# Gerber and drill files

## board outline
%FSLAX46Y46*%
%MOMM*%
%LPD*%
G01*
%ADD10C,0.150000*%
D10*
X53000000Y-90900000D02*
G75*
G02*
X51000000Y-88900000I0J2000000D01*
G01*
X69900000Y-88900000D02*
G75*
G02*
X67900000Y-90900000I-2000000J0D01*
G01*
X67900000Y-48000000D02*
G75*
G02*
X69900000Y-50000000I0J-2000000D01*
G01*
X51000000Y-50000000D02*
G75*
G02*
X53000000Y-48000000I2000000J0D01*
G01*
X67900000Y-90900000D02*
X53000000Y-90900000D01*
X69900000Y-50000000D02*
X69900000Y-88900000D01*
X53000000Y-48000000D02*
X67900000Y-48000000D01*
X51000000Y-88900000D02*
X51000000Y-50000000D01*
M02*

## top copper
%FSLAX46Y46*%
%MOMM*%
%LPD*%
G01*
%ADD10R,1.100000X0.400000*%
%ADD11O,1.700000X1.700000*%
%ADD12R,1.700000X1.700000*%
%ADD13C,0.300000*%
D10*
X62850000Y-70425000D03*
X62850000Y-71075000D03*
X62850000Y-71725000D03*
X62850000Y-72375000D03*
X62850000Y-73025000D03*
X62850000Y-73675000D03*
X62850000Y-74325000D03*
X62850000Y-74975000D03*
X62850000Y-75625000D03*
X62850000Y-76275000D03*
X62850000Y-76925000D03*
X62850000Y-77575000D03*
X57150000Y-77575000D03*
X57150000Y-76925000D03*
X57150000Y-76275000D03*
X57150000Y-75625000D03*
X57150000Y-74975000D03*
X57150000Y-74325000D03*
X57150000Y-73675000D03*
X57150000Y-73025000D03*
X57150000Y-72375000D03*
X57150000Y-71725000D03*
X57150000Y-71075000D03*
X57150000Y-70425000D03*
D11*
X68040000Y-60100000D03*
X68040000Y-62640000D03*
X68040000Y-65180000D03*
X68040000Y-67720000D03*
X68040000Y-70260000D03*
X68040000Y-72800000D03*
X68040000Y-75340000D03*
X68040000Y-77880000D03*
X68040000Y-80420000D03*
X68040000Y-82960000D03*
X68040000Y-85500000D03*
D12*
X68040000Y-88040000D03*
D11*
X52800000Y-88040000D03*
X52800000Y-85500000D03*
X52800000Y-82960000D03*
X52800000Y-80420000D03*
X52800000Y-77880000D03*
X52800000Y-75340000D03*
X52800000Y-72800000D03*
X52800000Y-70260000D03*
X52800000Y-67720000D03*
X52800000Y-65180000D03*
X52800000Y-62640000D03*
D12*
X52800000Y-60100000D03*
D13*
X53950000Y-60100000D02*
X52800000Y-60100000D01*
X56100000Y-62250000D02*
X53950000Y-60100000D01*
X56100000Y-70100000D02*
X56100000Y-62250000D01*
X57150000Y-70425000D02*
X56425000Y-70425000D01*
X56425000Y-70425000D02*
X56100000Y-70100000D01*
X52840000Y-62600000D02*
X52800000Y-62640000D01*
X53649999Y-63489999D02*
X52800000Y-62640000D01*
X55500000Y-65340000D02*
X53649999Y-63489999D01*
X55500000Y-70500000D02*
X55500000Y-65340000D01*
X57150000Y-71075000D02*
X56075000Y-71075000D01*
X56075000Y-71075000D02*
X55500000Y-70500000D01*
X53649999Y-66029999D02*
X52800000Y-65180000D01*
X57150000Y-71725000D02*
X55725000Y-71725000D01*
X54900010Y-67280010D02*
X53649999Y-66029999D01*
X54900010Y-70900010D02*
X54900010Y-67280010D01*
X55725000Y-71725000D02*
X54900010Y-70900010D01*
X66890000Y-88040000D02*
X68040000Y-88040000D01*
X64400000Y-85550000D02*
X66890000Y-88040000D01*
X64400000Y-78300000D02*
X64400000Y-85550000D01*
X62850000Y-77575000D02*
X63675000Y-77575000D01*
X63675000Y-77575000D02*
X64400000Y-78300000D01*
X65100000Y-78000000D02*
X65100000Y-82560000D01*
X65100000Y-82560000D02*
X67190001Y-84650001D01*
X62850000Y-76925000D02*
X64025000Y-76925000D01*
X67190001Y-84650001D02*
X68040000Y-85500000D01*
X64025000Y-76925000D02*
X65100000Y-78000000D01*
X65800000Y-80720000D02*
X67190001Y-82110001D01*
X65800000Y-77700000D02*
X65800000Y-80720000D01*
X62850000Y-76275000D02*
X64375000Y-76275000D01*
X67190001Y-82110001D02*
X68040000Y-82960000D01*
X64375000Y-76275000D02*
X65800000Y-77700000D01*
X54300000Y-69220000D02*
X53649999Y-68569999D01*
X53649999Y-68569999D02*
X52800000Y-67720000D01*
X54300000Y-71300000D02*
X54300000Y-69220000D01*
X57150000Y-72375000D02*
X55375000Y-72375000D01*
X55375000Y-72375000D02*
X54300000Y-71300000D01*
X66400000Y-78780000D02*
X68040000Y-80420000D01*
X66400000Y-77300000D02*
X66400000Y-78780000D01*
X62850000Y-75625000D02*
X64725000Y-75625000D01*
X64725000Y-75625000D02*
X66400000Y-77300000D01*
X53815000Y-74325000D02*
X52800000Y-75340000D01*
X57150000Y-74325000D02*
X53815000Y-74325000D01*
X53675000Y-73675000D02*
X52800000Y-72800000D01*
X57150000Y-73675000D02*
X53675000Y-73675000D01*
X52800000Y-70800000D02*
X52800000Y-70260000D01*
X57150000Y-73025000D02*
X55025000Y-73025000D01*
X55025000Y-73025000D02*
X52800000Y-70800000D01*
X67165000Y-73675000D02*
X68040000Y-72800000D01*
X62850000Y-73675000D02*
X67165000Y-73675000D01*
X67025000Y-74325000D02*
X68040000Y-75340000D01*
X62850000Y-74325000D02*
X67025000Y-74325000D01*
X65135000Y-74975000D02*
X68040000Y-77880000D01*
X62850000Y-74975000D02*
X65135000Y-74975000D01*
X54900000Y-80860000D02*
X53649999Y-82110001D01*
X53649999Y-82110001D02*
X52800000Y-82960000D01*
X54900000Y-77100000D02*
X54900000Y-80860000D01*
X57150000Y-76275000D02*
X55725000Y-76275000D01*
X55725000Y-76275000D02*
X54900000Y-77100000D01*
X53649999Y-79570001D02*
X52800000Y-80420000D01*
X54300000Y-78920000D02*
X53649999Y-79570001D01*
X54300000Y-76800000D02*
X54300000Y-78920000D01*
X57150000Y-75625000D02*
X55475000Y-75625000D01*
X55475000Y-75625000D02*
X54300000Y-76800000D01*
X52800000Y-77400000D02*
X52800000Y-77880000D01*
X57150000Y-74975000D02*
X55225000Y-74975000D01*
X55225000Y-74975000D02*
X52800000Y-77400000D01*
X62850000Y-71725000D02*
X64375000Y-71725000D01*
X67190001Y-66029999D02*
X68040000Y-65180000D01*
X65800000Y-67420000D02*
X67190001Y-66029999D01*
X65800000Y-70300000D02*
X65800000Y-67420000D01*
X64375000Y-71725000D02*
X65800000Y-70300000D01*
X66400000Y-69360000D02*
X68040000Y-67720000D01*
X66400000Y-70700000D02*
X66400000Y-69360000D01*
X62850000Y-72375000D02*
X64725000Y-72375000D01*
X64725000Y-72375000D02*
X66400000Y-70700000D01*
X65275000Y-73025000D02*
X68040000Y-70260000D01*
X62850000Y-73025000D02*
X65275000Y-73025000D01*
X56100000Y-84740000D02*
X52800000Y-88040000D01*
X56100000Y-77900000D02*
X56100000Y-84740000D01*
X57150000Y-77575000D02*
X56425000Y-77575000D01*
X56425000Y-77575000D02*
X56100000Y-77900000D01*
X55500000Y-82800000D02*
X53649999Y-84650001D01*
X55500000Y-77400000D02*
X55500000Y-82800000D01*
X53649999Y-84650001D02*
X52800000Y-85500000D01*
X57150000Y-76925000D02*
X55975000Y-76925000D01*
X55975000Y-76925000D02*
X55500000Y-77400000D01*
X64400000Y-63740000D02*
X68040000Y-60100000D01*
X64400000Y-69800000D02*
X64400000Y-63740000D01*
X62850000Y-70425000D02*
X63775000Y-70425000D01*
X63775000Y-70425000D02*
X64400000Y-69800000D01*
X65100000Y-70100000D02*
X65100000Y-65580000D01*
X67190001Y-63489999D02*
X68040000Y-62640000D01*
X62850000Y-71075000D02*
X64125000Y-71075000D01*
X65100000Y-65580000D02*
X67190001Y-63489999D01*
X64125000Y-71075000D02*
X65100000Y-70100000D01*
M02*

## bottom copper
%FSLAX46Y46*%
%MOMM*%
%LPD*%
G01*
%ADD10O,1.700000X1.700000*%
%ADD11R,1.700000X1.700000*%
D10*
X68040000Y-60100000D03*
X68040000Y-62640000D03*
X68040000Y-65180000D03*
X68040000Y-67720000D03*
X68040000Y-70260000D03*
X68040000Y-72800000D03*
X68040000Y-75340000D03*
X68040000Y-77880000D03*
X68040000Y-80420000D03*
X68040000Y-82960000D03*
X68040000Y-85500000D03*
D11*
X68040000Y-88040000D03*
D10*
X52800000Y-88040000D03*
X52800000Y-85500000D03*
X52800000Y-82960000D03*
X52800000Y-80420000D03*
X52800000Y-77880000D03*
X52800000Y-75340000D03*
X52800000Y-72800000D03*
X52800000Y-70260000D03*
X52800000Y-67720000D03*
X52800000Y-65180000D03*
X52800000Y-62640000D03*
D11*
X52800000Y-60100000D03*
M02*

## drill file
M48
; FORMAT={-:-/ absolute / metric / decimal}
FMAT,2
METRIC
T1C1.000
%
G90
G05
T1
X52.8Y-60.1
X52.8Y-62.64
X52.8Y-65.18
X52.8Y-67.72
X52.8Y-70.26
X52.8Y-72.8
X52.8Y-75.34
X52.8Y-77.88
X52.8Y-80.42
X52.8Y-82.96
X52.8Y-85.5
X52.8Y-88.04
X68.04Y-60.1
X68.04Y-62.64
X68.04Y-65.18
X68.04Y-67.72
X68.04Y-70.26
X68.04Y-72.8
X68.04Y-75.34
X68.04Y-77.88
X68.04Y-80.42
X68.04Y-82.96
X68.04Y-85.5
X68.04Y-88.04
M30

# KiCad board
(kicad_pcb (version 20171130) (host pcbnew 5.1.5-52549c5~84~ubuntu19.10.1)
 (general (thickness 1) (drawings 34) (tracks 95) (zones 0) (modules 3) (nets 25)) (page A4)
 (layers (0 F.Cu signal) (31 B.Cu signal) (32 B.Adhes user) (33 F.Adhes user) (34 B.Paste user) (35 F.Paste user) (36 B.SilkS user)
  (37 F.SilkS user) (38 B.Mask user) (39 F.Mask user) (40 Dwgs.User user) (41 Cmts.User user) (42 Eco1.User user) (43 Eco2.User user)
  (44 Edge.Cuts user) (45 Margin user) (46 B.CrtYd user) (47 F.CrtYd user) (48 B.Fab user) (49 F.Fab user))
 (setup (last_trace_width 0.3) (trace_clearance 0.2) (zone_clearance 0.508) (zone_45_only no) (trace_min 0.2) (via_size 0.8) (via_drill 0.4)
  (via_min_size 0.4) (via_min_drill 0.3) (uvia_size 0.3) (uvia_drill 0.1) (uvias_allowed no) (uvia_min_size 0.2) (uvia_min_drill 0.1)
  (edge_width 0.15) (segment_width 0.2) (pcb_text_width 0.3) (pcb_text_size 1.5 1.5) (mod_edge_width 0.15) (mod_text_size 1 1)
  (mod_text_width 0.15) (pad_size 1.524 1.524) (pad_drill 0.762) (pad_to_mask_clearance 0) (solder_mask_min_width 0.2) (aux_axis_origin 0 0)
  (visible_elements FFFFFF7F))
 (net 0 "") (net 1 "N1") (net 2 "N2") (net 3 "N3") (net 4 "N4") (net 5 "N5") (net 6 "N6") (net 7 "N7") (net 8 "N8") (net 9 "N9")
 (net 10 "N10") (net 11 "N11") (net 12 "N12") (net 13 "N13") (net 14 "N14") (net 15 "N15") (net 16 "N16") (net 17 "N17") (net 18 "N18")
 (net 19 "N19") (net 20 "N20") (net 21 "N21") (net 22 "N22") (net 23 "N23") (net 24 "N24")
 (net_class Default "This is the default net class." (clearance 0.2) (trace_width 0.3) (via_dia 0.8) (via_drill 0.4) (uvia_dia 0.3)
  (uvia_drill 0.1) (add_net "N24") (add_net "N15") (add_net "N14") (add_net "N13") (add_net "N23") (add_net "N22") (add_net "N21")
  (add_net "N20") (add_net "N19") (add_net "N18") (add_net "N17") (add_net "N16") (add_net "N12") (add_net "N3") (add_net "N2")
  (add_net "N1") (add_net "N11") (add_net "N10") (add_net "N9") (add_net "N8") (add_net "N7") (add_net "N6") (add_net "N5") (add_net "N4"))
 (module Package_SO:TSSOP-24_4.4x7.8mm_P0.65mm (layer F.Cu) (at 60 74)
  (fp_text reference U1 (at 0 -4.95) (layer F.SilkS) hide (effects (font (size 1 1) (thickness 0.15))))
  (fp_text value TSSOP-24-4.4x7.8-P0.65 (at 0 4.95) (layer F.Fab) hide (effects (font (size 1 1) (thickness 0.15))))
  (pad 24 smd rect (at 2.85 -3.575) (size 1.1 0.4) (layers F.Cu F.Paste F.Mask) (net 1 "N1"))
  (pad 23 smd rect (at 2.85 -2.925) (size 1.1 0.4) (layers F.Cu F.Paste F.Mask) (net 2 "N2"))
  (pad 22 smd rect (at 2.85 -2.275) (size 1.1 0.4) (layers F.Cu F.Paste F.Mask) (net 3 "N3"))
  (pad 21 smd rect (at 2.85 -1.625) (size 1.1 0.4) (layers F.Cu F.Paste F.Mask) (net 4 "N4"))
  (pad 20 smd rect (at 2.85 -0.975) (size 1.1 0.4) (layers F.Cu F.Paste F.Mask) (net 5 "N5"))
  (pad 19 smd rect (at 2.85 -0.325) (size 1.1 0.4) (layers F.Cu F.Paste F.Mask) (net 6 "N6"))
  (pad 18 smd rect (at 2.85 0.325) (size 1.1 0.4) (layers F.Cu F.Paste F.Mask) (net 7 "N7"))
  (pad 17 smd rect (at 2.85 0.975) (size 1.1 0.4) (layers F.Cu F.Paste F.Mask) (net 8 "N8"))
  (pad 16 smd rect (at 2.85 1.625) (size 1.1 0.4) (layers F.Cu F.Paste F.Mask) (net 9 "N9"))
  (pad 15 smd rect (at 2.85 2.275) (size 1.1 0.4) (layers F.Cu F.Paste F.Mask) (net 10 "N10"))
  (pad 14 smd rect (at 2.85 2.925) (size 1.1 0.4) (layers F.Cu F.Paste F.Mask) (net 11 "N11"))
  (pad 13 smd rect (at 2.85 3.575) (size 1.1 0.4) (layers F.Cu F.Paste F.Mask) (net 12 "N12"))
  (pad 12 smd rect (at -2.85 3.575) (size 1.1 0.4) (layers F.Cu F.Paste F.Mask) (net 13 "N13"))
  (pad 11 smd rect (at -2.85 2.925) (size 1.1 0.4) (layers F.Cu F.Paste F.Mask) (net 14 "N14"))
  (pad 10 smd rect (at -2.85 2.275) (size 1.1 0.4) (layers F.Cu F.Paste F.Mask) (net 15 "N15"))
  (pad 9 smd rect (at -2.85 1.625) (size 1.1 0.4) (layers F.Cu F.Paste F.Mask) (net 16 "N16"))
  (pad 8 smd rect (at -2.85 0.975) (size 1.1 0.4) (layers F.Cu F.Paste F.Mask) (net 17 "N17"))
  (pad 7 smd rect (at -2.85 0.325) (size 1.1 0.4) (layers F.Cu F.Paste F.Mask) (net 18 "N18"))
  (pad 6 smd rect (at -2.85 -0.325) (size 1.1 0.4) (layers F.Cu F.Paste F.Mask) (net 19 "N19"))
  (pad 5 smd rect (at -2.85 -0.975) (size 1.1 0.4) (layers F.Cu F.Paste F.Mask) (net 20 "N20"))
  (pad 4 smd rect (at -2.85 -1.625) (size 1.1 0.4) (layers F.Cu F.Paste F.Mask) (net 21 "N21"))
  (pad 3 smd rect (at -2.85 -2.275) (size 1.1 0.4) (layers F.Cu F.Paste F.Mask) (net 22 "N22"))
  (pad 2 smd rect (at -2.85 -2.925) (size 1.1 0.4) (layers F.Cu F.Paste F.Mask) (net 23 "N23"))
  (pad 1 smd rect (at -2.85 -3.575) (size 1.1 0.4) (layers F.Cu F.Paste F.Mask) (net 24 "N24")))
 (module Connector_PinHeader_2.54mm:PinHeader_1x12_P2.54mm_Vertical (layer F.Cu) (at 68.04 88.04 180)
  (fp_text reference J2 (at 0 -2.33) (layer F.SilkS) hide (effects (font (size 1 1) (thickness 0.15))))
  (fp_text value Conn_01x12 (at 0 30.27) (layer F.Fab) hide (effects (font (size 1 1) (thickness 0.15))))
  (pad 12 thru_hole oval (at 0 27.94 180) (size 1.7 1.7) (drill 1) (layers *.Cu *.Mask) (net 1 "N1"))
  (pad 11 thru_hole oval (at 0 25.4 180) (size 1.7 1.7) (drill 1) (layers *.Cu *.Mask) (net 2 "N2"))
  (pad 10 thru_hole oval (at 0 22.86 180) (size 1.7 1.7) (drill 1) (layers *.Cu *.Mask) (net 3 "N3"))
  (pad 9 thru_hole oval (at 0 20.32 180) (size 1.7 1.7) (drill 1) (layers *.Cu *.Mask) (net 4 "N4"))
  (pad 8 thru_hole oval (at 0 17.78 180) (size 1.7 1.7) (drill 1) (layers *.Cu *.Mask) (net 5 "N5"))
  (pad 7 thru_hole oval (at 0 15.24 180) (size 1.7 1.7) (drill 1) (layers *.Cu *.Mask) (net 6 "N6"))
  (pad 6 thru_hole oval (at 0 12.7 180) (size 1.7 1.7) (drill 1) (layers *.Cu *.Mask) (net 7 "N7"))
  (pad 5 thru_hole oval (at 0 10.16 180) (size 1.7 1.7) (drill 1) (layers *.Cu *.Mask) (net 8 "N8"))
  (pad 4 thru_hole oval (at 0 7.62 180) (size 1.7 1.7) (drill 1) (layers *.Cu *.Mask) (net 9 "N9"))
  (pad 3 thru_hole oval (at 0 5.08 180) (size 1.7 1.7) (drill 1) (layers *.Cu *.Mask) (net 10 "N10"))
  (pad 2 thru_hole oval (at 0 2.54 180) (size 1.7 1.7) (drill 1) (layers *.Cu *.Mask) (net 11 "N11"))
  (pad 1 thru_hole rect (at 0 0 180) (size 1.7 1.7) (drill 1) (layers *.Cu *.Mask) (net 12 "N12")))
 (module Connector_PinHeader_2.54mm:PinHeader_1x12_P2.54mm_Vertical (layer F.Cu) (at 52.8 60.1)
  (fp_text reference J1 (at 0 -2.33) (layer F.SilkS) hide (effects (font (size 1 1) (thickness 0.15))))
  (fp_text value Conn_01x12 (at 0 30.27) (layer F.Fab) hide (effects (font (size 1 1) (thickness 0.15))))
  (pad 12 thru_hole oval (at 0 27.94) (size 1.7 1.7) (drill 1) (layers *.Cu *.Mask) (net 13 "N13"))
  (pad 11 thru_hole oval (at 0 25.4) (size 1.7 1.7) (drill 1) (layers *.Cu *.Mask) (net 14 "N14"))
  (pad 10 thru_hole oval (at 0 22.86) (size 1.7 1.7) (drill 1) (layers *.Cu *.Mask) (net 15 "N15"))
  (pad 9 thru_hole oval (at 0 20.32) (size 1.7 1.7) (drill 1) (layers *.Cu *.Mask) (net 16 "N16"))
  (pad 8 thru_hole oval (at 0 17.78) (size 1.7 1.7) (drill 1) (layers *.Cu *.Mask) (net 17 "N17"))
  (pad 7 thru_hole oval (at 0 15.24) (size 1.7 1.7) (drill 1) (layers *.Cu *.Mask) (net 18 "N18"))
  (pad 6 thru_hole oval (at 0 12.7) (size 1.7 1.7) (drill 1) (layers *.Cu *.Mask) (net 19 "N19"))
  (pad 5 thru_hole oval (at 0 10.16) (size 1.7 1.7) (drill 1) (layers *.Cu *.Mask) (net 20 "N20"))
  (pad 4 thru_hole oval (at 0 7.62) (size 1.7 1.7) (drill 1) (layers *.Cu *.Mask) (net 21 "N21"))
  (pad 3 thru_hole oval (at 0 5.08) (size 1.7 1.7) (drill 1) (layers *.Cu *.Mask) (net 22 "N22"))
  (pad 2 thru_hole oval (at 0 2.54) (size 1.7 1.7) (drill 1) (layers *.Cu *.Mask) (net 23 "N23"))
  (pad 1 thru_hole rect (at 0 0) (size 1.7 1.7) (drill 1) (layers *.Cu *.Mask) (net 24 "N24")))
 (gr_arc (start 53 88.9) (end 51 88.9) (angle -90) (layer Edge.Cuts) (width 0.15))
 (gr_arc (start 67.9 88.9) (end 67.9 90.9) (angle -90) (layer Edge.Cuts) (width 0.15))
 (gr_arc (start 67.9 50) (end 69.9 50) (angle -90) (layer Edge.Cuts) (width 0.15))
 (gr_arc (start 53 50) (end 53 48) (angle -90) (layer Edge.Cuts) (width 0.15))
 (gr_line (start 67.9 90.9) (end 53 90.9) (layer Edge.Cuts) (width 0.15))
 (gr_line (start 69.9 50) (end 69.9 88.9) (layer Edge.Cuts) (width 0.15))
 (gr_line (start 53 48) (end 67.9 48) (layer Edge.Cuts) (width 0.15))
 (gr_line (start 51 88.9) (end 51 50) (layer Edge.Cuts) (width 0.15))
 (segment (start 53.95 60.1) (end 52.8 60.1) (width 0.3) (layer F.Cu) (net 24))
 (segment (start 56.1 62.25) (end 53.95 60.1) (width 0.3) (layer F.Cu) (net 24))
 (segment (start 56.1 70.1) (end 56.1 62.25) (width 0.3) (layer F.Cu) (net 24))
 (segment (start 57.15 70.425) (end 56.425 70.425) (width 0.3) (layer F.Cu) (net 24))
 (segment (start 56.425 70.425) (end 56.1 70.1) (width 0.3) (layer F.Cu) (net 24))
 (segment (start 52.84 62.6) (end 52.8 62.64) (width 0.3) (layer F.Cu) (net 23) (status 30))
 (segment (start 53.649999 63.489999) (end 52.8 62.64) (width 0.3) (layer F.Cu) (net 23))
 (segment (start 55.5 65.34) (end 53.649999 63.489999) (width 0.3) (layer F.Cu) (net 23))
 (segment (start 55.5 70.5) (end 55.5 65.34) (width 0.3) (layer F.Cu) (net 23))
 (segment (start 57.15 71.075) (end 56.075 71.075) (width 0.3) (layer F.Cu) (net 23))
 (segment (start 56.075 71.075) (end 55.5 70.5) (width 0.3) (layer F.Cu) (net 23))
 (segment (start 53.649999 66.029999) (end 52.8 65.18) (width 0.3) (layer F.Cu) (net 22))
 (segment (start 57.15 71.725) (end 55.725 71.725) (width 0.3) (layer F.Cu) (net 22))
 (segment (start 54.90001 67.28001) (end 53.649999 66.029999) (width 0.3) (layer F.Cu) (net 22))
 (segment (start 54.90001 70.90001) (end 54.90001 67.28001) (width 0.3) (layer F.Cu) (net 22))
 (segment (start 55.725 71.725) (end 54.90001 70.90001) (width 0.3) (layer F.Cu) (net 22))
 (segment (start 66.89 88.04) (end 68.04 88.04) (width 0.3) (layer F.Cu) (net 12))
 (segment (start 64.4 85.55) (end 66.89 88.04) (width 0.3) (layer F.Cu) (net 12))
 (segment (start 64.4 78.3) (end 64.4 85.55) (width 0.3) (layer F.Cu) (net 12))
 (segment (start 62.85 77.575) (end 63.675 77.575) (width 0.3) (layer F.Cu) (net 12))
 (segment (start 63.675 77.575) (end 64.4 78.3) (width 0.3) (layer F.Cu) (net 12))
 (segment (start 65.1 78) (end 65.1 82.56) (width 0.3) (layer F.Cu) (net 11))
 (segment (start 65.1 82.56) (end 67.190001 84.650001) (width 0.3) (layer F.Cu) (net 11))
 (segment (start 62.85 76.925) (end 64.025 76.925) (width 0.3) (layer F.Cu) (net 11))
 (segment (start 67.190001 84.650001) (end 68.04 85.5) (width 0.3) (layer F.Cu) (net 11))
 (segment (start 64.025 76.925) (end 65.1 78) (width 0.3) (layer F.Cu) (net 11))
 (segment (start 65.8 80.72) (end 67.190001 82.110001) (width 0.3) (layer F.Cu) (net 10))
 (segment (start 65.8 77.7) (end 65.8 80.72) (width 0.3) (layer F.Cu) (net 10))
 (segment (start 62.85 76.275) (end 64.375 76.275) (width 0.3) (layer F.Cu) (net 10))
 (segment (start 67.190001 82.110001) (end 68.04 82.96) (width 0.3) (layer F.Cu) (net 10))
 (segment (start 64.375 76.275) (end 65.8 77.7) (width 0.3) (layer F.Cu) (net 10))
 (segment (start 54.3 69.22) (end 53.649999 68.569999) (width 0.3) (layer F.Cu) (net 21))
 (segment (start 53.649999 68.569999) (end 52.8 67.72) (width 0.3) (layer F.Cu) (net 21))
 (segment (start 54.3 71.3) (end 54.3 69.22) (width 0.3) (layer F.Cu) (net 21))
 (segment (start 57.15 72.375) (end 55.375 72.375) (width 0.3) (layer F.Cu) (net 21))
 (segment (start 55.375 72.375) (end 54.3 71.3) (width 0.3) (layer F.Cu) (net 21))
 (segment (start 66.4 78.78) (end 68.04 80.42) (width 0.3) (layer F.Cu) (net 9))
 (segment (start 66.4 77.3) (end 66.4 78.78) (width 0.3) (layer F.Cu) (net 9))
 (segment (start 62.85 75.625) (end 64.725 75.625) (width 0.3) (layer F.Cu) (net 9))
 (segment (start 64.725 75.625) (end 66.4 77.3) (width 0.3) (layer F.Cu) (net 9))
 (segment (start 53.815 74.325) (end 52.8 75.34) (width 0.3) (layer F.Cu) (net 18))
 (segment (start 57.15 74.325) (end 53.815 74.325) (width 0.3) (layer F.Cu) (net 18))
 (segment (start 53.675 73.675) (end 52.8 72.8) (width 0.3) (layer F.Cu) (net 19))
 (segment (start 57.15 73.675) (end 53.675 73.675) (width 0.3) (layer F.Cu) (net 19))
 (segment (start 52.8 70.8) (end 52.8 70.26) (width 0.3) (layer F.Cu) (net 20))
 (segment (start 57.15 73.025) (end 55.025 73.025) (width 0.3) (layer F.Cu) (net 20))
 (segment (start 55.025 73.025) (end 52.8 70.8) (width 0.3) (layer F.Cu) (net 20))
 (segment (start 67.165 73.675) (end 68.04 72.8) (width 0.3) (layer F.Cu) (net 6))
 (segment (start 62.85 73.675) (end 67.165 73.675) (width 0.3) (layer F.Cu) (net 6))
 (segment (start 67.025 74.325) (end 68.04 75.34) (width 0.3) (layer F.Cu) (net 7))
 (segment (start 62.85 74.325) (end 67.025 74.325) (width 0.3) (layer F.Cu) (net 7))
 (segment (start 65.135 74.975) (end 68.04 77.88) (width 0.3) (layer F.Cu) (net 8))
 (segment (start 62.85 74.975) (end 65.135 74.975) (width 0.3) (layer F.Cu) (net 8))
 (segment (start 54.9 80.86) (end 53.649999 82.110001) (width 0.3) (layer F.Cu) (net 15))
 (segment (start 53.649999 82.110001) (end 52.8 82.96) (width 0.3) (layer F.Cu) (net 15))
 (segment (start 54.9 77.1) (end 54.9 80.86) (width 0.3) (layer F.Cu) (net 15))
 (segment (start 57.15 76.275) (end 55.725 76.275) (width 0.3) (layer F.Cu) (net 15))
 (segment (start 55.725 76.275) (end 54.9 77.1) (width 0.3) (layer F.Cu) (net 15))
 (segment (start 53.649999 79.570001) (end 52.8 80.42) (width 0.3) (layer F.Cu) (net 16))
 (segment (start 54.3 78.92) (end 53.649999 79.570001) (width 0.3) (layer F.Cu) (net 16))
 (segment (start 54.3 76.8) (end 54.3 78.92) (width 0.3) (layer F.Cu) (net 16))
 (segment (start 57.15 75.625) (end 55.475 75.625) (width 0.3) (layer F.Cu) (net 16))
 (segment (start 55.475 75.625) (end 54.3 76.8) (width 0.3) (layer F.Cu) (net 16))
 (segment (start 52.8 77.4) (end 52.8 77.88) (width 0.3) (layer F.Cu) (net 17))
 (segment (start 57.15 74.975) (end 55.225 74.975) (width 0.3) (layer F.Cu) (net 17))
 (segment (start 55.225 74.975) (end 52.8 77.4) (width 0.3) (layer F.Cu) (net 17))
 (segment (start 62.85 71.725) (end 64.375 71.725) (width 0.3) (layer F.Cu) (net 3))
 (segment (start 67.190001 66.029999) (end 68.04 65.18) (width 0.3) (layer F.Cu) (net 3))
 (segment (start 65.8 67.42) (end 67.190001 66.029999) (width 0.3) (layer F.Cu) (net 3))
 (segment (start 65.8 70.3) (end 65.8 67.42) (width 0.3) (layer F.Cu) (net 3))
 (segment (start 64.375 71.725) (end 65.8 70.3) (width 0.3) (layer F.Cu) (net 3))
 (segment (start 66.4 69.36) (end 68.04 67.72) (width 0.3) (layer F.Cu) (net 4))
 (segment (start 66.4 70.7) (end 66.4 69.36) (width 0.3) (layer F.Cu) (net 4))
 (segment (start 62.85 72.375) (end 64.725 72.375) (width 0.3) (layer F.Cu) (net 4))
 (segment (start 64.725 72.375) (end 66.4 70.7) (width 0.3) (layer F.Cu) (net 4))
 (segment (start 65.275 73.025) (end 68.04 70.26) (width 0.3) (layer F.Cu) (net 5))
 (segment (start 62.85 73.025) (end 65.275 73.025) (width 0.3) (layer F.Cu) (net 5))
 (segment (start 56.1 84.74) (end 52.8 88.04) (width 0.3) (layer F.Cu) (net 13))
 (segment (start 56.1 77.9) (end 56.1 84.74) (width 0.3) (layer F.Cu) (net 13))
 (segment (start 57.15 77.575) (end 56.425 77.575) (width 0.3) (layer F.Cu) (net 13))
 (segment (start 56.425 77.575) (end 56.1 77.9) (width 0.3) (layer F.Cu) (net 13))
 (segment (start 55.5 82.8) (end 53.649999 84.650001) (width 0.3) (layer F.Cu) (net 14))
 (segment (start 55.5 77.4) (end 55.5 82.8) (width 0.3) (layer F.Cu) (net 14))
 (segment (start 53.649999 84.650001) (end 52.8 85.5) (width 0.3) (layer F.Cu) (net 14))
 (segment (start 57.15 76.925) (end 55.975 76.925) (width 0.3) (layer F.Cu) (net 14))
 (segment (start 55.975 76.925) (end 55.5 77.4) (width 0.3) (layer F.Cu) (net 14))
 (segment (start 64.4 63.74) (end 68.04 60.1) (width 0.3) (layer F.Cu) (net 1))
 (segment (start 64.4 69.8) (end 64.4 63.74) (width 0.3) (layer F.Cu) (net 1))
 (segment (start 62.85 70.425) (end 63.775 70.425) (width 0.3) (layer F.Cu) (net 1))
 (segment (start 63.775 70.425) (end 64.4 69.8) (width 0.3) (layer F.Cu) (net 1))
 (segment (start 65.1 70.1) (end 65.1 65.58) (width 0.3) (layer F.Cu) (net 2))
 (segment (start 67.190001 63.489999) (end 68.04 62.64) (width 0.3) (layer F.Cu) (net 2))
 (segment (start 62.85 71.075) (end 64.125 71.075) (width 0.3) (layer F.Cu) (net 2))
 (segment (start 65.1 65.58) (end 67.190001 63.489999) (width 0.3) (layer F.Cu) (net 2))
 (segment (start 64.125 71.075) (end 65.1 70.1) (width 0.3) (layer F.Cu) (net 2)))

